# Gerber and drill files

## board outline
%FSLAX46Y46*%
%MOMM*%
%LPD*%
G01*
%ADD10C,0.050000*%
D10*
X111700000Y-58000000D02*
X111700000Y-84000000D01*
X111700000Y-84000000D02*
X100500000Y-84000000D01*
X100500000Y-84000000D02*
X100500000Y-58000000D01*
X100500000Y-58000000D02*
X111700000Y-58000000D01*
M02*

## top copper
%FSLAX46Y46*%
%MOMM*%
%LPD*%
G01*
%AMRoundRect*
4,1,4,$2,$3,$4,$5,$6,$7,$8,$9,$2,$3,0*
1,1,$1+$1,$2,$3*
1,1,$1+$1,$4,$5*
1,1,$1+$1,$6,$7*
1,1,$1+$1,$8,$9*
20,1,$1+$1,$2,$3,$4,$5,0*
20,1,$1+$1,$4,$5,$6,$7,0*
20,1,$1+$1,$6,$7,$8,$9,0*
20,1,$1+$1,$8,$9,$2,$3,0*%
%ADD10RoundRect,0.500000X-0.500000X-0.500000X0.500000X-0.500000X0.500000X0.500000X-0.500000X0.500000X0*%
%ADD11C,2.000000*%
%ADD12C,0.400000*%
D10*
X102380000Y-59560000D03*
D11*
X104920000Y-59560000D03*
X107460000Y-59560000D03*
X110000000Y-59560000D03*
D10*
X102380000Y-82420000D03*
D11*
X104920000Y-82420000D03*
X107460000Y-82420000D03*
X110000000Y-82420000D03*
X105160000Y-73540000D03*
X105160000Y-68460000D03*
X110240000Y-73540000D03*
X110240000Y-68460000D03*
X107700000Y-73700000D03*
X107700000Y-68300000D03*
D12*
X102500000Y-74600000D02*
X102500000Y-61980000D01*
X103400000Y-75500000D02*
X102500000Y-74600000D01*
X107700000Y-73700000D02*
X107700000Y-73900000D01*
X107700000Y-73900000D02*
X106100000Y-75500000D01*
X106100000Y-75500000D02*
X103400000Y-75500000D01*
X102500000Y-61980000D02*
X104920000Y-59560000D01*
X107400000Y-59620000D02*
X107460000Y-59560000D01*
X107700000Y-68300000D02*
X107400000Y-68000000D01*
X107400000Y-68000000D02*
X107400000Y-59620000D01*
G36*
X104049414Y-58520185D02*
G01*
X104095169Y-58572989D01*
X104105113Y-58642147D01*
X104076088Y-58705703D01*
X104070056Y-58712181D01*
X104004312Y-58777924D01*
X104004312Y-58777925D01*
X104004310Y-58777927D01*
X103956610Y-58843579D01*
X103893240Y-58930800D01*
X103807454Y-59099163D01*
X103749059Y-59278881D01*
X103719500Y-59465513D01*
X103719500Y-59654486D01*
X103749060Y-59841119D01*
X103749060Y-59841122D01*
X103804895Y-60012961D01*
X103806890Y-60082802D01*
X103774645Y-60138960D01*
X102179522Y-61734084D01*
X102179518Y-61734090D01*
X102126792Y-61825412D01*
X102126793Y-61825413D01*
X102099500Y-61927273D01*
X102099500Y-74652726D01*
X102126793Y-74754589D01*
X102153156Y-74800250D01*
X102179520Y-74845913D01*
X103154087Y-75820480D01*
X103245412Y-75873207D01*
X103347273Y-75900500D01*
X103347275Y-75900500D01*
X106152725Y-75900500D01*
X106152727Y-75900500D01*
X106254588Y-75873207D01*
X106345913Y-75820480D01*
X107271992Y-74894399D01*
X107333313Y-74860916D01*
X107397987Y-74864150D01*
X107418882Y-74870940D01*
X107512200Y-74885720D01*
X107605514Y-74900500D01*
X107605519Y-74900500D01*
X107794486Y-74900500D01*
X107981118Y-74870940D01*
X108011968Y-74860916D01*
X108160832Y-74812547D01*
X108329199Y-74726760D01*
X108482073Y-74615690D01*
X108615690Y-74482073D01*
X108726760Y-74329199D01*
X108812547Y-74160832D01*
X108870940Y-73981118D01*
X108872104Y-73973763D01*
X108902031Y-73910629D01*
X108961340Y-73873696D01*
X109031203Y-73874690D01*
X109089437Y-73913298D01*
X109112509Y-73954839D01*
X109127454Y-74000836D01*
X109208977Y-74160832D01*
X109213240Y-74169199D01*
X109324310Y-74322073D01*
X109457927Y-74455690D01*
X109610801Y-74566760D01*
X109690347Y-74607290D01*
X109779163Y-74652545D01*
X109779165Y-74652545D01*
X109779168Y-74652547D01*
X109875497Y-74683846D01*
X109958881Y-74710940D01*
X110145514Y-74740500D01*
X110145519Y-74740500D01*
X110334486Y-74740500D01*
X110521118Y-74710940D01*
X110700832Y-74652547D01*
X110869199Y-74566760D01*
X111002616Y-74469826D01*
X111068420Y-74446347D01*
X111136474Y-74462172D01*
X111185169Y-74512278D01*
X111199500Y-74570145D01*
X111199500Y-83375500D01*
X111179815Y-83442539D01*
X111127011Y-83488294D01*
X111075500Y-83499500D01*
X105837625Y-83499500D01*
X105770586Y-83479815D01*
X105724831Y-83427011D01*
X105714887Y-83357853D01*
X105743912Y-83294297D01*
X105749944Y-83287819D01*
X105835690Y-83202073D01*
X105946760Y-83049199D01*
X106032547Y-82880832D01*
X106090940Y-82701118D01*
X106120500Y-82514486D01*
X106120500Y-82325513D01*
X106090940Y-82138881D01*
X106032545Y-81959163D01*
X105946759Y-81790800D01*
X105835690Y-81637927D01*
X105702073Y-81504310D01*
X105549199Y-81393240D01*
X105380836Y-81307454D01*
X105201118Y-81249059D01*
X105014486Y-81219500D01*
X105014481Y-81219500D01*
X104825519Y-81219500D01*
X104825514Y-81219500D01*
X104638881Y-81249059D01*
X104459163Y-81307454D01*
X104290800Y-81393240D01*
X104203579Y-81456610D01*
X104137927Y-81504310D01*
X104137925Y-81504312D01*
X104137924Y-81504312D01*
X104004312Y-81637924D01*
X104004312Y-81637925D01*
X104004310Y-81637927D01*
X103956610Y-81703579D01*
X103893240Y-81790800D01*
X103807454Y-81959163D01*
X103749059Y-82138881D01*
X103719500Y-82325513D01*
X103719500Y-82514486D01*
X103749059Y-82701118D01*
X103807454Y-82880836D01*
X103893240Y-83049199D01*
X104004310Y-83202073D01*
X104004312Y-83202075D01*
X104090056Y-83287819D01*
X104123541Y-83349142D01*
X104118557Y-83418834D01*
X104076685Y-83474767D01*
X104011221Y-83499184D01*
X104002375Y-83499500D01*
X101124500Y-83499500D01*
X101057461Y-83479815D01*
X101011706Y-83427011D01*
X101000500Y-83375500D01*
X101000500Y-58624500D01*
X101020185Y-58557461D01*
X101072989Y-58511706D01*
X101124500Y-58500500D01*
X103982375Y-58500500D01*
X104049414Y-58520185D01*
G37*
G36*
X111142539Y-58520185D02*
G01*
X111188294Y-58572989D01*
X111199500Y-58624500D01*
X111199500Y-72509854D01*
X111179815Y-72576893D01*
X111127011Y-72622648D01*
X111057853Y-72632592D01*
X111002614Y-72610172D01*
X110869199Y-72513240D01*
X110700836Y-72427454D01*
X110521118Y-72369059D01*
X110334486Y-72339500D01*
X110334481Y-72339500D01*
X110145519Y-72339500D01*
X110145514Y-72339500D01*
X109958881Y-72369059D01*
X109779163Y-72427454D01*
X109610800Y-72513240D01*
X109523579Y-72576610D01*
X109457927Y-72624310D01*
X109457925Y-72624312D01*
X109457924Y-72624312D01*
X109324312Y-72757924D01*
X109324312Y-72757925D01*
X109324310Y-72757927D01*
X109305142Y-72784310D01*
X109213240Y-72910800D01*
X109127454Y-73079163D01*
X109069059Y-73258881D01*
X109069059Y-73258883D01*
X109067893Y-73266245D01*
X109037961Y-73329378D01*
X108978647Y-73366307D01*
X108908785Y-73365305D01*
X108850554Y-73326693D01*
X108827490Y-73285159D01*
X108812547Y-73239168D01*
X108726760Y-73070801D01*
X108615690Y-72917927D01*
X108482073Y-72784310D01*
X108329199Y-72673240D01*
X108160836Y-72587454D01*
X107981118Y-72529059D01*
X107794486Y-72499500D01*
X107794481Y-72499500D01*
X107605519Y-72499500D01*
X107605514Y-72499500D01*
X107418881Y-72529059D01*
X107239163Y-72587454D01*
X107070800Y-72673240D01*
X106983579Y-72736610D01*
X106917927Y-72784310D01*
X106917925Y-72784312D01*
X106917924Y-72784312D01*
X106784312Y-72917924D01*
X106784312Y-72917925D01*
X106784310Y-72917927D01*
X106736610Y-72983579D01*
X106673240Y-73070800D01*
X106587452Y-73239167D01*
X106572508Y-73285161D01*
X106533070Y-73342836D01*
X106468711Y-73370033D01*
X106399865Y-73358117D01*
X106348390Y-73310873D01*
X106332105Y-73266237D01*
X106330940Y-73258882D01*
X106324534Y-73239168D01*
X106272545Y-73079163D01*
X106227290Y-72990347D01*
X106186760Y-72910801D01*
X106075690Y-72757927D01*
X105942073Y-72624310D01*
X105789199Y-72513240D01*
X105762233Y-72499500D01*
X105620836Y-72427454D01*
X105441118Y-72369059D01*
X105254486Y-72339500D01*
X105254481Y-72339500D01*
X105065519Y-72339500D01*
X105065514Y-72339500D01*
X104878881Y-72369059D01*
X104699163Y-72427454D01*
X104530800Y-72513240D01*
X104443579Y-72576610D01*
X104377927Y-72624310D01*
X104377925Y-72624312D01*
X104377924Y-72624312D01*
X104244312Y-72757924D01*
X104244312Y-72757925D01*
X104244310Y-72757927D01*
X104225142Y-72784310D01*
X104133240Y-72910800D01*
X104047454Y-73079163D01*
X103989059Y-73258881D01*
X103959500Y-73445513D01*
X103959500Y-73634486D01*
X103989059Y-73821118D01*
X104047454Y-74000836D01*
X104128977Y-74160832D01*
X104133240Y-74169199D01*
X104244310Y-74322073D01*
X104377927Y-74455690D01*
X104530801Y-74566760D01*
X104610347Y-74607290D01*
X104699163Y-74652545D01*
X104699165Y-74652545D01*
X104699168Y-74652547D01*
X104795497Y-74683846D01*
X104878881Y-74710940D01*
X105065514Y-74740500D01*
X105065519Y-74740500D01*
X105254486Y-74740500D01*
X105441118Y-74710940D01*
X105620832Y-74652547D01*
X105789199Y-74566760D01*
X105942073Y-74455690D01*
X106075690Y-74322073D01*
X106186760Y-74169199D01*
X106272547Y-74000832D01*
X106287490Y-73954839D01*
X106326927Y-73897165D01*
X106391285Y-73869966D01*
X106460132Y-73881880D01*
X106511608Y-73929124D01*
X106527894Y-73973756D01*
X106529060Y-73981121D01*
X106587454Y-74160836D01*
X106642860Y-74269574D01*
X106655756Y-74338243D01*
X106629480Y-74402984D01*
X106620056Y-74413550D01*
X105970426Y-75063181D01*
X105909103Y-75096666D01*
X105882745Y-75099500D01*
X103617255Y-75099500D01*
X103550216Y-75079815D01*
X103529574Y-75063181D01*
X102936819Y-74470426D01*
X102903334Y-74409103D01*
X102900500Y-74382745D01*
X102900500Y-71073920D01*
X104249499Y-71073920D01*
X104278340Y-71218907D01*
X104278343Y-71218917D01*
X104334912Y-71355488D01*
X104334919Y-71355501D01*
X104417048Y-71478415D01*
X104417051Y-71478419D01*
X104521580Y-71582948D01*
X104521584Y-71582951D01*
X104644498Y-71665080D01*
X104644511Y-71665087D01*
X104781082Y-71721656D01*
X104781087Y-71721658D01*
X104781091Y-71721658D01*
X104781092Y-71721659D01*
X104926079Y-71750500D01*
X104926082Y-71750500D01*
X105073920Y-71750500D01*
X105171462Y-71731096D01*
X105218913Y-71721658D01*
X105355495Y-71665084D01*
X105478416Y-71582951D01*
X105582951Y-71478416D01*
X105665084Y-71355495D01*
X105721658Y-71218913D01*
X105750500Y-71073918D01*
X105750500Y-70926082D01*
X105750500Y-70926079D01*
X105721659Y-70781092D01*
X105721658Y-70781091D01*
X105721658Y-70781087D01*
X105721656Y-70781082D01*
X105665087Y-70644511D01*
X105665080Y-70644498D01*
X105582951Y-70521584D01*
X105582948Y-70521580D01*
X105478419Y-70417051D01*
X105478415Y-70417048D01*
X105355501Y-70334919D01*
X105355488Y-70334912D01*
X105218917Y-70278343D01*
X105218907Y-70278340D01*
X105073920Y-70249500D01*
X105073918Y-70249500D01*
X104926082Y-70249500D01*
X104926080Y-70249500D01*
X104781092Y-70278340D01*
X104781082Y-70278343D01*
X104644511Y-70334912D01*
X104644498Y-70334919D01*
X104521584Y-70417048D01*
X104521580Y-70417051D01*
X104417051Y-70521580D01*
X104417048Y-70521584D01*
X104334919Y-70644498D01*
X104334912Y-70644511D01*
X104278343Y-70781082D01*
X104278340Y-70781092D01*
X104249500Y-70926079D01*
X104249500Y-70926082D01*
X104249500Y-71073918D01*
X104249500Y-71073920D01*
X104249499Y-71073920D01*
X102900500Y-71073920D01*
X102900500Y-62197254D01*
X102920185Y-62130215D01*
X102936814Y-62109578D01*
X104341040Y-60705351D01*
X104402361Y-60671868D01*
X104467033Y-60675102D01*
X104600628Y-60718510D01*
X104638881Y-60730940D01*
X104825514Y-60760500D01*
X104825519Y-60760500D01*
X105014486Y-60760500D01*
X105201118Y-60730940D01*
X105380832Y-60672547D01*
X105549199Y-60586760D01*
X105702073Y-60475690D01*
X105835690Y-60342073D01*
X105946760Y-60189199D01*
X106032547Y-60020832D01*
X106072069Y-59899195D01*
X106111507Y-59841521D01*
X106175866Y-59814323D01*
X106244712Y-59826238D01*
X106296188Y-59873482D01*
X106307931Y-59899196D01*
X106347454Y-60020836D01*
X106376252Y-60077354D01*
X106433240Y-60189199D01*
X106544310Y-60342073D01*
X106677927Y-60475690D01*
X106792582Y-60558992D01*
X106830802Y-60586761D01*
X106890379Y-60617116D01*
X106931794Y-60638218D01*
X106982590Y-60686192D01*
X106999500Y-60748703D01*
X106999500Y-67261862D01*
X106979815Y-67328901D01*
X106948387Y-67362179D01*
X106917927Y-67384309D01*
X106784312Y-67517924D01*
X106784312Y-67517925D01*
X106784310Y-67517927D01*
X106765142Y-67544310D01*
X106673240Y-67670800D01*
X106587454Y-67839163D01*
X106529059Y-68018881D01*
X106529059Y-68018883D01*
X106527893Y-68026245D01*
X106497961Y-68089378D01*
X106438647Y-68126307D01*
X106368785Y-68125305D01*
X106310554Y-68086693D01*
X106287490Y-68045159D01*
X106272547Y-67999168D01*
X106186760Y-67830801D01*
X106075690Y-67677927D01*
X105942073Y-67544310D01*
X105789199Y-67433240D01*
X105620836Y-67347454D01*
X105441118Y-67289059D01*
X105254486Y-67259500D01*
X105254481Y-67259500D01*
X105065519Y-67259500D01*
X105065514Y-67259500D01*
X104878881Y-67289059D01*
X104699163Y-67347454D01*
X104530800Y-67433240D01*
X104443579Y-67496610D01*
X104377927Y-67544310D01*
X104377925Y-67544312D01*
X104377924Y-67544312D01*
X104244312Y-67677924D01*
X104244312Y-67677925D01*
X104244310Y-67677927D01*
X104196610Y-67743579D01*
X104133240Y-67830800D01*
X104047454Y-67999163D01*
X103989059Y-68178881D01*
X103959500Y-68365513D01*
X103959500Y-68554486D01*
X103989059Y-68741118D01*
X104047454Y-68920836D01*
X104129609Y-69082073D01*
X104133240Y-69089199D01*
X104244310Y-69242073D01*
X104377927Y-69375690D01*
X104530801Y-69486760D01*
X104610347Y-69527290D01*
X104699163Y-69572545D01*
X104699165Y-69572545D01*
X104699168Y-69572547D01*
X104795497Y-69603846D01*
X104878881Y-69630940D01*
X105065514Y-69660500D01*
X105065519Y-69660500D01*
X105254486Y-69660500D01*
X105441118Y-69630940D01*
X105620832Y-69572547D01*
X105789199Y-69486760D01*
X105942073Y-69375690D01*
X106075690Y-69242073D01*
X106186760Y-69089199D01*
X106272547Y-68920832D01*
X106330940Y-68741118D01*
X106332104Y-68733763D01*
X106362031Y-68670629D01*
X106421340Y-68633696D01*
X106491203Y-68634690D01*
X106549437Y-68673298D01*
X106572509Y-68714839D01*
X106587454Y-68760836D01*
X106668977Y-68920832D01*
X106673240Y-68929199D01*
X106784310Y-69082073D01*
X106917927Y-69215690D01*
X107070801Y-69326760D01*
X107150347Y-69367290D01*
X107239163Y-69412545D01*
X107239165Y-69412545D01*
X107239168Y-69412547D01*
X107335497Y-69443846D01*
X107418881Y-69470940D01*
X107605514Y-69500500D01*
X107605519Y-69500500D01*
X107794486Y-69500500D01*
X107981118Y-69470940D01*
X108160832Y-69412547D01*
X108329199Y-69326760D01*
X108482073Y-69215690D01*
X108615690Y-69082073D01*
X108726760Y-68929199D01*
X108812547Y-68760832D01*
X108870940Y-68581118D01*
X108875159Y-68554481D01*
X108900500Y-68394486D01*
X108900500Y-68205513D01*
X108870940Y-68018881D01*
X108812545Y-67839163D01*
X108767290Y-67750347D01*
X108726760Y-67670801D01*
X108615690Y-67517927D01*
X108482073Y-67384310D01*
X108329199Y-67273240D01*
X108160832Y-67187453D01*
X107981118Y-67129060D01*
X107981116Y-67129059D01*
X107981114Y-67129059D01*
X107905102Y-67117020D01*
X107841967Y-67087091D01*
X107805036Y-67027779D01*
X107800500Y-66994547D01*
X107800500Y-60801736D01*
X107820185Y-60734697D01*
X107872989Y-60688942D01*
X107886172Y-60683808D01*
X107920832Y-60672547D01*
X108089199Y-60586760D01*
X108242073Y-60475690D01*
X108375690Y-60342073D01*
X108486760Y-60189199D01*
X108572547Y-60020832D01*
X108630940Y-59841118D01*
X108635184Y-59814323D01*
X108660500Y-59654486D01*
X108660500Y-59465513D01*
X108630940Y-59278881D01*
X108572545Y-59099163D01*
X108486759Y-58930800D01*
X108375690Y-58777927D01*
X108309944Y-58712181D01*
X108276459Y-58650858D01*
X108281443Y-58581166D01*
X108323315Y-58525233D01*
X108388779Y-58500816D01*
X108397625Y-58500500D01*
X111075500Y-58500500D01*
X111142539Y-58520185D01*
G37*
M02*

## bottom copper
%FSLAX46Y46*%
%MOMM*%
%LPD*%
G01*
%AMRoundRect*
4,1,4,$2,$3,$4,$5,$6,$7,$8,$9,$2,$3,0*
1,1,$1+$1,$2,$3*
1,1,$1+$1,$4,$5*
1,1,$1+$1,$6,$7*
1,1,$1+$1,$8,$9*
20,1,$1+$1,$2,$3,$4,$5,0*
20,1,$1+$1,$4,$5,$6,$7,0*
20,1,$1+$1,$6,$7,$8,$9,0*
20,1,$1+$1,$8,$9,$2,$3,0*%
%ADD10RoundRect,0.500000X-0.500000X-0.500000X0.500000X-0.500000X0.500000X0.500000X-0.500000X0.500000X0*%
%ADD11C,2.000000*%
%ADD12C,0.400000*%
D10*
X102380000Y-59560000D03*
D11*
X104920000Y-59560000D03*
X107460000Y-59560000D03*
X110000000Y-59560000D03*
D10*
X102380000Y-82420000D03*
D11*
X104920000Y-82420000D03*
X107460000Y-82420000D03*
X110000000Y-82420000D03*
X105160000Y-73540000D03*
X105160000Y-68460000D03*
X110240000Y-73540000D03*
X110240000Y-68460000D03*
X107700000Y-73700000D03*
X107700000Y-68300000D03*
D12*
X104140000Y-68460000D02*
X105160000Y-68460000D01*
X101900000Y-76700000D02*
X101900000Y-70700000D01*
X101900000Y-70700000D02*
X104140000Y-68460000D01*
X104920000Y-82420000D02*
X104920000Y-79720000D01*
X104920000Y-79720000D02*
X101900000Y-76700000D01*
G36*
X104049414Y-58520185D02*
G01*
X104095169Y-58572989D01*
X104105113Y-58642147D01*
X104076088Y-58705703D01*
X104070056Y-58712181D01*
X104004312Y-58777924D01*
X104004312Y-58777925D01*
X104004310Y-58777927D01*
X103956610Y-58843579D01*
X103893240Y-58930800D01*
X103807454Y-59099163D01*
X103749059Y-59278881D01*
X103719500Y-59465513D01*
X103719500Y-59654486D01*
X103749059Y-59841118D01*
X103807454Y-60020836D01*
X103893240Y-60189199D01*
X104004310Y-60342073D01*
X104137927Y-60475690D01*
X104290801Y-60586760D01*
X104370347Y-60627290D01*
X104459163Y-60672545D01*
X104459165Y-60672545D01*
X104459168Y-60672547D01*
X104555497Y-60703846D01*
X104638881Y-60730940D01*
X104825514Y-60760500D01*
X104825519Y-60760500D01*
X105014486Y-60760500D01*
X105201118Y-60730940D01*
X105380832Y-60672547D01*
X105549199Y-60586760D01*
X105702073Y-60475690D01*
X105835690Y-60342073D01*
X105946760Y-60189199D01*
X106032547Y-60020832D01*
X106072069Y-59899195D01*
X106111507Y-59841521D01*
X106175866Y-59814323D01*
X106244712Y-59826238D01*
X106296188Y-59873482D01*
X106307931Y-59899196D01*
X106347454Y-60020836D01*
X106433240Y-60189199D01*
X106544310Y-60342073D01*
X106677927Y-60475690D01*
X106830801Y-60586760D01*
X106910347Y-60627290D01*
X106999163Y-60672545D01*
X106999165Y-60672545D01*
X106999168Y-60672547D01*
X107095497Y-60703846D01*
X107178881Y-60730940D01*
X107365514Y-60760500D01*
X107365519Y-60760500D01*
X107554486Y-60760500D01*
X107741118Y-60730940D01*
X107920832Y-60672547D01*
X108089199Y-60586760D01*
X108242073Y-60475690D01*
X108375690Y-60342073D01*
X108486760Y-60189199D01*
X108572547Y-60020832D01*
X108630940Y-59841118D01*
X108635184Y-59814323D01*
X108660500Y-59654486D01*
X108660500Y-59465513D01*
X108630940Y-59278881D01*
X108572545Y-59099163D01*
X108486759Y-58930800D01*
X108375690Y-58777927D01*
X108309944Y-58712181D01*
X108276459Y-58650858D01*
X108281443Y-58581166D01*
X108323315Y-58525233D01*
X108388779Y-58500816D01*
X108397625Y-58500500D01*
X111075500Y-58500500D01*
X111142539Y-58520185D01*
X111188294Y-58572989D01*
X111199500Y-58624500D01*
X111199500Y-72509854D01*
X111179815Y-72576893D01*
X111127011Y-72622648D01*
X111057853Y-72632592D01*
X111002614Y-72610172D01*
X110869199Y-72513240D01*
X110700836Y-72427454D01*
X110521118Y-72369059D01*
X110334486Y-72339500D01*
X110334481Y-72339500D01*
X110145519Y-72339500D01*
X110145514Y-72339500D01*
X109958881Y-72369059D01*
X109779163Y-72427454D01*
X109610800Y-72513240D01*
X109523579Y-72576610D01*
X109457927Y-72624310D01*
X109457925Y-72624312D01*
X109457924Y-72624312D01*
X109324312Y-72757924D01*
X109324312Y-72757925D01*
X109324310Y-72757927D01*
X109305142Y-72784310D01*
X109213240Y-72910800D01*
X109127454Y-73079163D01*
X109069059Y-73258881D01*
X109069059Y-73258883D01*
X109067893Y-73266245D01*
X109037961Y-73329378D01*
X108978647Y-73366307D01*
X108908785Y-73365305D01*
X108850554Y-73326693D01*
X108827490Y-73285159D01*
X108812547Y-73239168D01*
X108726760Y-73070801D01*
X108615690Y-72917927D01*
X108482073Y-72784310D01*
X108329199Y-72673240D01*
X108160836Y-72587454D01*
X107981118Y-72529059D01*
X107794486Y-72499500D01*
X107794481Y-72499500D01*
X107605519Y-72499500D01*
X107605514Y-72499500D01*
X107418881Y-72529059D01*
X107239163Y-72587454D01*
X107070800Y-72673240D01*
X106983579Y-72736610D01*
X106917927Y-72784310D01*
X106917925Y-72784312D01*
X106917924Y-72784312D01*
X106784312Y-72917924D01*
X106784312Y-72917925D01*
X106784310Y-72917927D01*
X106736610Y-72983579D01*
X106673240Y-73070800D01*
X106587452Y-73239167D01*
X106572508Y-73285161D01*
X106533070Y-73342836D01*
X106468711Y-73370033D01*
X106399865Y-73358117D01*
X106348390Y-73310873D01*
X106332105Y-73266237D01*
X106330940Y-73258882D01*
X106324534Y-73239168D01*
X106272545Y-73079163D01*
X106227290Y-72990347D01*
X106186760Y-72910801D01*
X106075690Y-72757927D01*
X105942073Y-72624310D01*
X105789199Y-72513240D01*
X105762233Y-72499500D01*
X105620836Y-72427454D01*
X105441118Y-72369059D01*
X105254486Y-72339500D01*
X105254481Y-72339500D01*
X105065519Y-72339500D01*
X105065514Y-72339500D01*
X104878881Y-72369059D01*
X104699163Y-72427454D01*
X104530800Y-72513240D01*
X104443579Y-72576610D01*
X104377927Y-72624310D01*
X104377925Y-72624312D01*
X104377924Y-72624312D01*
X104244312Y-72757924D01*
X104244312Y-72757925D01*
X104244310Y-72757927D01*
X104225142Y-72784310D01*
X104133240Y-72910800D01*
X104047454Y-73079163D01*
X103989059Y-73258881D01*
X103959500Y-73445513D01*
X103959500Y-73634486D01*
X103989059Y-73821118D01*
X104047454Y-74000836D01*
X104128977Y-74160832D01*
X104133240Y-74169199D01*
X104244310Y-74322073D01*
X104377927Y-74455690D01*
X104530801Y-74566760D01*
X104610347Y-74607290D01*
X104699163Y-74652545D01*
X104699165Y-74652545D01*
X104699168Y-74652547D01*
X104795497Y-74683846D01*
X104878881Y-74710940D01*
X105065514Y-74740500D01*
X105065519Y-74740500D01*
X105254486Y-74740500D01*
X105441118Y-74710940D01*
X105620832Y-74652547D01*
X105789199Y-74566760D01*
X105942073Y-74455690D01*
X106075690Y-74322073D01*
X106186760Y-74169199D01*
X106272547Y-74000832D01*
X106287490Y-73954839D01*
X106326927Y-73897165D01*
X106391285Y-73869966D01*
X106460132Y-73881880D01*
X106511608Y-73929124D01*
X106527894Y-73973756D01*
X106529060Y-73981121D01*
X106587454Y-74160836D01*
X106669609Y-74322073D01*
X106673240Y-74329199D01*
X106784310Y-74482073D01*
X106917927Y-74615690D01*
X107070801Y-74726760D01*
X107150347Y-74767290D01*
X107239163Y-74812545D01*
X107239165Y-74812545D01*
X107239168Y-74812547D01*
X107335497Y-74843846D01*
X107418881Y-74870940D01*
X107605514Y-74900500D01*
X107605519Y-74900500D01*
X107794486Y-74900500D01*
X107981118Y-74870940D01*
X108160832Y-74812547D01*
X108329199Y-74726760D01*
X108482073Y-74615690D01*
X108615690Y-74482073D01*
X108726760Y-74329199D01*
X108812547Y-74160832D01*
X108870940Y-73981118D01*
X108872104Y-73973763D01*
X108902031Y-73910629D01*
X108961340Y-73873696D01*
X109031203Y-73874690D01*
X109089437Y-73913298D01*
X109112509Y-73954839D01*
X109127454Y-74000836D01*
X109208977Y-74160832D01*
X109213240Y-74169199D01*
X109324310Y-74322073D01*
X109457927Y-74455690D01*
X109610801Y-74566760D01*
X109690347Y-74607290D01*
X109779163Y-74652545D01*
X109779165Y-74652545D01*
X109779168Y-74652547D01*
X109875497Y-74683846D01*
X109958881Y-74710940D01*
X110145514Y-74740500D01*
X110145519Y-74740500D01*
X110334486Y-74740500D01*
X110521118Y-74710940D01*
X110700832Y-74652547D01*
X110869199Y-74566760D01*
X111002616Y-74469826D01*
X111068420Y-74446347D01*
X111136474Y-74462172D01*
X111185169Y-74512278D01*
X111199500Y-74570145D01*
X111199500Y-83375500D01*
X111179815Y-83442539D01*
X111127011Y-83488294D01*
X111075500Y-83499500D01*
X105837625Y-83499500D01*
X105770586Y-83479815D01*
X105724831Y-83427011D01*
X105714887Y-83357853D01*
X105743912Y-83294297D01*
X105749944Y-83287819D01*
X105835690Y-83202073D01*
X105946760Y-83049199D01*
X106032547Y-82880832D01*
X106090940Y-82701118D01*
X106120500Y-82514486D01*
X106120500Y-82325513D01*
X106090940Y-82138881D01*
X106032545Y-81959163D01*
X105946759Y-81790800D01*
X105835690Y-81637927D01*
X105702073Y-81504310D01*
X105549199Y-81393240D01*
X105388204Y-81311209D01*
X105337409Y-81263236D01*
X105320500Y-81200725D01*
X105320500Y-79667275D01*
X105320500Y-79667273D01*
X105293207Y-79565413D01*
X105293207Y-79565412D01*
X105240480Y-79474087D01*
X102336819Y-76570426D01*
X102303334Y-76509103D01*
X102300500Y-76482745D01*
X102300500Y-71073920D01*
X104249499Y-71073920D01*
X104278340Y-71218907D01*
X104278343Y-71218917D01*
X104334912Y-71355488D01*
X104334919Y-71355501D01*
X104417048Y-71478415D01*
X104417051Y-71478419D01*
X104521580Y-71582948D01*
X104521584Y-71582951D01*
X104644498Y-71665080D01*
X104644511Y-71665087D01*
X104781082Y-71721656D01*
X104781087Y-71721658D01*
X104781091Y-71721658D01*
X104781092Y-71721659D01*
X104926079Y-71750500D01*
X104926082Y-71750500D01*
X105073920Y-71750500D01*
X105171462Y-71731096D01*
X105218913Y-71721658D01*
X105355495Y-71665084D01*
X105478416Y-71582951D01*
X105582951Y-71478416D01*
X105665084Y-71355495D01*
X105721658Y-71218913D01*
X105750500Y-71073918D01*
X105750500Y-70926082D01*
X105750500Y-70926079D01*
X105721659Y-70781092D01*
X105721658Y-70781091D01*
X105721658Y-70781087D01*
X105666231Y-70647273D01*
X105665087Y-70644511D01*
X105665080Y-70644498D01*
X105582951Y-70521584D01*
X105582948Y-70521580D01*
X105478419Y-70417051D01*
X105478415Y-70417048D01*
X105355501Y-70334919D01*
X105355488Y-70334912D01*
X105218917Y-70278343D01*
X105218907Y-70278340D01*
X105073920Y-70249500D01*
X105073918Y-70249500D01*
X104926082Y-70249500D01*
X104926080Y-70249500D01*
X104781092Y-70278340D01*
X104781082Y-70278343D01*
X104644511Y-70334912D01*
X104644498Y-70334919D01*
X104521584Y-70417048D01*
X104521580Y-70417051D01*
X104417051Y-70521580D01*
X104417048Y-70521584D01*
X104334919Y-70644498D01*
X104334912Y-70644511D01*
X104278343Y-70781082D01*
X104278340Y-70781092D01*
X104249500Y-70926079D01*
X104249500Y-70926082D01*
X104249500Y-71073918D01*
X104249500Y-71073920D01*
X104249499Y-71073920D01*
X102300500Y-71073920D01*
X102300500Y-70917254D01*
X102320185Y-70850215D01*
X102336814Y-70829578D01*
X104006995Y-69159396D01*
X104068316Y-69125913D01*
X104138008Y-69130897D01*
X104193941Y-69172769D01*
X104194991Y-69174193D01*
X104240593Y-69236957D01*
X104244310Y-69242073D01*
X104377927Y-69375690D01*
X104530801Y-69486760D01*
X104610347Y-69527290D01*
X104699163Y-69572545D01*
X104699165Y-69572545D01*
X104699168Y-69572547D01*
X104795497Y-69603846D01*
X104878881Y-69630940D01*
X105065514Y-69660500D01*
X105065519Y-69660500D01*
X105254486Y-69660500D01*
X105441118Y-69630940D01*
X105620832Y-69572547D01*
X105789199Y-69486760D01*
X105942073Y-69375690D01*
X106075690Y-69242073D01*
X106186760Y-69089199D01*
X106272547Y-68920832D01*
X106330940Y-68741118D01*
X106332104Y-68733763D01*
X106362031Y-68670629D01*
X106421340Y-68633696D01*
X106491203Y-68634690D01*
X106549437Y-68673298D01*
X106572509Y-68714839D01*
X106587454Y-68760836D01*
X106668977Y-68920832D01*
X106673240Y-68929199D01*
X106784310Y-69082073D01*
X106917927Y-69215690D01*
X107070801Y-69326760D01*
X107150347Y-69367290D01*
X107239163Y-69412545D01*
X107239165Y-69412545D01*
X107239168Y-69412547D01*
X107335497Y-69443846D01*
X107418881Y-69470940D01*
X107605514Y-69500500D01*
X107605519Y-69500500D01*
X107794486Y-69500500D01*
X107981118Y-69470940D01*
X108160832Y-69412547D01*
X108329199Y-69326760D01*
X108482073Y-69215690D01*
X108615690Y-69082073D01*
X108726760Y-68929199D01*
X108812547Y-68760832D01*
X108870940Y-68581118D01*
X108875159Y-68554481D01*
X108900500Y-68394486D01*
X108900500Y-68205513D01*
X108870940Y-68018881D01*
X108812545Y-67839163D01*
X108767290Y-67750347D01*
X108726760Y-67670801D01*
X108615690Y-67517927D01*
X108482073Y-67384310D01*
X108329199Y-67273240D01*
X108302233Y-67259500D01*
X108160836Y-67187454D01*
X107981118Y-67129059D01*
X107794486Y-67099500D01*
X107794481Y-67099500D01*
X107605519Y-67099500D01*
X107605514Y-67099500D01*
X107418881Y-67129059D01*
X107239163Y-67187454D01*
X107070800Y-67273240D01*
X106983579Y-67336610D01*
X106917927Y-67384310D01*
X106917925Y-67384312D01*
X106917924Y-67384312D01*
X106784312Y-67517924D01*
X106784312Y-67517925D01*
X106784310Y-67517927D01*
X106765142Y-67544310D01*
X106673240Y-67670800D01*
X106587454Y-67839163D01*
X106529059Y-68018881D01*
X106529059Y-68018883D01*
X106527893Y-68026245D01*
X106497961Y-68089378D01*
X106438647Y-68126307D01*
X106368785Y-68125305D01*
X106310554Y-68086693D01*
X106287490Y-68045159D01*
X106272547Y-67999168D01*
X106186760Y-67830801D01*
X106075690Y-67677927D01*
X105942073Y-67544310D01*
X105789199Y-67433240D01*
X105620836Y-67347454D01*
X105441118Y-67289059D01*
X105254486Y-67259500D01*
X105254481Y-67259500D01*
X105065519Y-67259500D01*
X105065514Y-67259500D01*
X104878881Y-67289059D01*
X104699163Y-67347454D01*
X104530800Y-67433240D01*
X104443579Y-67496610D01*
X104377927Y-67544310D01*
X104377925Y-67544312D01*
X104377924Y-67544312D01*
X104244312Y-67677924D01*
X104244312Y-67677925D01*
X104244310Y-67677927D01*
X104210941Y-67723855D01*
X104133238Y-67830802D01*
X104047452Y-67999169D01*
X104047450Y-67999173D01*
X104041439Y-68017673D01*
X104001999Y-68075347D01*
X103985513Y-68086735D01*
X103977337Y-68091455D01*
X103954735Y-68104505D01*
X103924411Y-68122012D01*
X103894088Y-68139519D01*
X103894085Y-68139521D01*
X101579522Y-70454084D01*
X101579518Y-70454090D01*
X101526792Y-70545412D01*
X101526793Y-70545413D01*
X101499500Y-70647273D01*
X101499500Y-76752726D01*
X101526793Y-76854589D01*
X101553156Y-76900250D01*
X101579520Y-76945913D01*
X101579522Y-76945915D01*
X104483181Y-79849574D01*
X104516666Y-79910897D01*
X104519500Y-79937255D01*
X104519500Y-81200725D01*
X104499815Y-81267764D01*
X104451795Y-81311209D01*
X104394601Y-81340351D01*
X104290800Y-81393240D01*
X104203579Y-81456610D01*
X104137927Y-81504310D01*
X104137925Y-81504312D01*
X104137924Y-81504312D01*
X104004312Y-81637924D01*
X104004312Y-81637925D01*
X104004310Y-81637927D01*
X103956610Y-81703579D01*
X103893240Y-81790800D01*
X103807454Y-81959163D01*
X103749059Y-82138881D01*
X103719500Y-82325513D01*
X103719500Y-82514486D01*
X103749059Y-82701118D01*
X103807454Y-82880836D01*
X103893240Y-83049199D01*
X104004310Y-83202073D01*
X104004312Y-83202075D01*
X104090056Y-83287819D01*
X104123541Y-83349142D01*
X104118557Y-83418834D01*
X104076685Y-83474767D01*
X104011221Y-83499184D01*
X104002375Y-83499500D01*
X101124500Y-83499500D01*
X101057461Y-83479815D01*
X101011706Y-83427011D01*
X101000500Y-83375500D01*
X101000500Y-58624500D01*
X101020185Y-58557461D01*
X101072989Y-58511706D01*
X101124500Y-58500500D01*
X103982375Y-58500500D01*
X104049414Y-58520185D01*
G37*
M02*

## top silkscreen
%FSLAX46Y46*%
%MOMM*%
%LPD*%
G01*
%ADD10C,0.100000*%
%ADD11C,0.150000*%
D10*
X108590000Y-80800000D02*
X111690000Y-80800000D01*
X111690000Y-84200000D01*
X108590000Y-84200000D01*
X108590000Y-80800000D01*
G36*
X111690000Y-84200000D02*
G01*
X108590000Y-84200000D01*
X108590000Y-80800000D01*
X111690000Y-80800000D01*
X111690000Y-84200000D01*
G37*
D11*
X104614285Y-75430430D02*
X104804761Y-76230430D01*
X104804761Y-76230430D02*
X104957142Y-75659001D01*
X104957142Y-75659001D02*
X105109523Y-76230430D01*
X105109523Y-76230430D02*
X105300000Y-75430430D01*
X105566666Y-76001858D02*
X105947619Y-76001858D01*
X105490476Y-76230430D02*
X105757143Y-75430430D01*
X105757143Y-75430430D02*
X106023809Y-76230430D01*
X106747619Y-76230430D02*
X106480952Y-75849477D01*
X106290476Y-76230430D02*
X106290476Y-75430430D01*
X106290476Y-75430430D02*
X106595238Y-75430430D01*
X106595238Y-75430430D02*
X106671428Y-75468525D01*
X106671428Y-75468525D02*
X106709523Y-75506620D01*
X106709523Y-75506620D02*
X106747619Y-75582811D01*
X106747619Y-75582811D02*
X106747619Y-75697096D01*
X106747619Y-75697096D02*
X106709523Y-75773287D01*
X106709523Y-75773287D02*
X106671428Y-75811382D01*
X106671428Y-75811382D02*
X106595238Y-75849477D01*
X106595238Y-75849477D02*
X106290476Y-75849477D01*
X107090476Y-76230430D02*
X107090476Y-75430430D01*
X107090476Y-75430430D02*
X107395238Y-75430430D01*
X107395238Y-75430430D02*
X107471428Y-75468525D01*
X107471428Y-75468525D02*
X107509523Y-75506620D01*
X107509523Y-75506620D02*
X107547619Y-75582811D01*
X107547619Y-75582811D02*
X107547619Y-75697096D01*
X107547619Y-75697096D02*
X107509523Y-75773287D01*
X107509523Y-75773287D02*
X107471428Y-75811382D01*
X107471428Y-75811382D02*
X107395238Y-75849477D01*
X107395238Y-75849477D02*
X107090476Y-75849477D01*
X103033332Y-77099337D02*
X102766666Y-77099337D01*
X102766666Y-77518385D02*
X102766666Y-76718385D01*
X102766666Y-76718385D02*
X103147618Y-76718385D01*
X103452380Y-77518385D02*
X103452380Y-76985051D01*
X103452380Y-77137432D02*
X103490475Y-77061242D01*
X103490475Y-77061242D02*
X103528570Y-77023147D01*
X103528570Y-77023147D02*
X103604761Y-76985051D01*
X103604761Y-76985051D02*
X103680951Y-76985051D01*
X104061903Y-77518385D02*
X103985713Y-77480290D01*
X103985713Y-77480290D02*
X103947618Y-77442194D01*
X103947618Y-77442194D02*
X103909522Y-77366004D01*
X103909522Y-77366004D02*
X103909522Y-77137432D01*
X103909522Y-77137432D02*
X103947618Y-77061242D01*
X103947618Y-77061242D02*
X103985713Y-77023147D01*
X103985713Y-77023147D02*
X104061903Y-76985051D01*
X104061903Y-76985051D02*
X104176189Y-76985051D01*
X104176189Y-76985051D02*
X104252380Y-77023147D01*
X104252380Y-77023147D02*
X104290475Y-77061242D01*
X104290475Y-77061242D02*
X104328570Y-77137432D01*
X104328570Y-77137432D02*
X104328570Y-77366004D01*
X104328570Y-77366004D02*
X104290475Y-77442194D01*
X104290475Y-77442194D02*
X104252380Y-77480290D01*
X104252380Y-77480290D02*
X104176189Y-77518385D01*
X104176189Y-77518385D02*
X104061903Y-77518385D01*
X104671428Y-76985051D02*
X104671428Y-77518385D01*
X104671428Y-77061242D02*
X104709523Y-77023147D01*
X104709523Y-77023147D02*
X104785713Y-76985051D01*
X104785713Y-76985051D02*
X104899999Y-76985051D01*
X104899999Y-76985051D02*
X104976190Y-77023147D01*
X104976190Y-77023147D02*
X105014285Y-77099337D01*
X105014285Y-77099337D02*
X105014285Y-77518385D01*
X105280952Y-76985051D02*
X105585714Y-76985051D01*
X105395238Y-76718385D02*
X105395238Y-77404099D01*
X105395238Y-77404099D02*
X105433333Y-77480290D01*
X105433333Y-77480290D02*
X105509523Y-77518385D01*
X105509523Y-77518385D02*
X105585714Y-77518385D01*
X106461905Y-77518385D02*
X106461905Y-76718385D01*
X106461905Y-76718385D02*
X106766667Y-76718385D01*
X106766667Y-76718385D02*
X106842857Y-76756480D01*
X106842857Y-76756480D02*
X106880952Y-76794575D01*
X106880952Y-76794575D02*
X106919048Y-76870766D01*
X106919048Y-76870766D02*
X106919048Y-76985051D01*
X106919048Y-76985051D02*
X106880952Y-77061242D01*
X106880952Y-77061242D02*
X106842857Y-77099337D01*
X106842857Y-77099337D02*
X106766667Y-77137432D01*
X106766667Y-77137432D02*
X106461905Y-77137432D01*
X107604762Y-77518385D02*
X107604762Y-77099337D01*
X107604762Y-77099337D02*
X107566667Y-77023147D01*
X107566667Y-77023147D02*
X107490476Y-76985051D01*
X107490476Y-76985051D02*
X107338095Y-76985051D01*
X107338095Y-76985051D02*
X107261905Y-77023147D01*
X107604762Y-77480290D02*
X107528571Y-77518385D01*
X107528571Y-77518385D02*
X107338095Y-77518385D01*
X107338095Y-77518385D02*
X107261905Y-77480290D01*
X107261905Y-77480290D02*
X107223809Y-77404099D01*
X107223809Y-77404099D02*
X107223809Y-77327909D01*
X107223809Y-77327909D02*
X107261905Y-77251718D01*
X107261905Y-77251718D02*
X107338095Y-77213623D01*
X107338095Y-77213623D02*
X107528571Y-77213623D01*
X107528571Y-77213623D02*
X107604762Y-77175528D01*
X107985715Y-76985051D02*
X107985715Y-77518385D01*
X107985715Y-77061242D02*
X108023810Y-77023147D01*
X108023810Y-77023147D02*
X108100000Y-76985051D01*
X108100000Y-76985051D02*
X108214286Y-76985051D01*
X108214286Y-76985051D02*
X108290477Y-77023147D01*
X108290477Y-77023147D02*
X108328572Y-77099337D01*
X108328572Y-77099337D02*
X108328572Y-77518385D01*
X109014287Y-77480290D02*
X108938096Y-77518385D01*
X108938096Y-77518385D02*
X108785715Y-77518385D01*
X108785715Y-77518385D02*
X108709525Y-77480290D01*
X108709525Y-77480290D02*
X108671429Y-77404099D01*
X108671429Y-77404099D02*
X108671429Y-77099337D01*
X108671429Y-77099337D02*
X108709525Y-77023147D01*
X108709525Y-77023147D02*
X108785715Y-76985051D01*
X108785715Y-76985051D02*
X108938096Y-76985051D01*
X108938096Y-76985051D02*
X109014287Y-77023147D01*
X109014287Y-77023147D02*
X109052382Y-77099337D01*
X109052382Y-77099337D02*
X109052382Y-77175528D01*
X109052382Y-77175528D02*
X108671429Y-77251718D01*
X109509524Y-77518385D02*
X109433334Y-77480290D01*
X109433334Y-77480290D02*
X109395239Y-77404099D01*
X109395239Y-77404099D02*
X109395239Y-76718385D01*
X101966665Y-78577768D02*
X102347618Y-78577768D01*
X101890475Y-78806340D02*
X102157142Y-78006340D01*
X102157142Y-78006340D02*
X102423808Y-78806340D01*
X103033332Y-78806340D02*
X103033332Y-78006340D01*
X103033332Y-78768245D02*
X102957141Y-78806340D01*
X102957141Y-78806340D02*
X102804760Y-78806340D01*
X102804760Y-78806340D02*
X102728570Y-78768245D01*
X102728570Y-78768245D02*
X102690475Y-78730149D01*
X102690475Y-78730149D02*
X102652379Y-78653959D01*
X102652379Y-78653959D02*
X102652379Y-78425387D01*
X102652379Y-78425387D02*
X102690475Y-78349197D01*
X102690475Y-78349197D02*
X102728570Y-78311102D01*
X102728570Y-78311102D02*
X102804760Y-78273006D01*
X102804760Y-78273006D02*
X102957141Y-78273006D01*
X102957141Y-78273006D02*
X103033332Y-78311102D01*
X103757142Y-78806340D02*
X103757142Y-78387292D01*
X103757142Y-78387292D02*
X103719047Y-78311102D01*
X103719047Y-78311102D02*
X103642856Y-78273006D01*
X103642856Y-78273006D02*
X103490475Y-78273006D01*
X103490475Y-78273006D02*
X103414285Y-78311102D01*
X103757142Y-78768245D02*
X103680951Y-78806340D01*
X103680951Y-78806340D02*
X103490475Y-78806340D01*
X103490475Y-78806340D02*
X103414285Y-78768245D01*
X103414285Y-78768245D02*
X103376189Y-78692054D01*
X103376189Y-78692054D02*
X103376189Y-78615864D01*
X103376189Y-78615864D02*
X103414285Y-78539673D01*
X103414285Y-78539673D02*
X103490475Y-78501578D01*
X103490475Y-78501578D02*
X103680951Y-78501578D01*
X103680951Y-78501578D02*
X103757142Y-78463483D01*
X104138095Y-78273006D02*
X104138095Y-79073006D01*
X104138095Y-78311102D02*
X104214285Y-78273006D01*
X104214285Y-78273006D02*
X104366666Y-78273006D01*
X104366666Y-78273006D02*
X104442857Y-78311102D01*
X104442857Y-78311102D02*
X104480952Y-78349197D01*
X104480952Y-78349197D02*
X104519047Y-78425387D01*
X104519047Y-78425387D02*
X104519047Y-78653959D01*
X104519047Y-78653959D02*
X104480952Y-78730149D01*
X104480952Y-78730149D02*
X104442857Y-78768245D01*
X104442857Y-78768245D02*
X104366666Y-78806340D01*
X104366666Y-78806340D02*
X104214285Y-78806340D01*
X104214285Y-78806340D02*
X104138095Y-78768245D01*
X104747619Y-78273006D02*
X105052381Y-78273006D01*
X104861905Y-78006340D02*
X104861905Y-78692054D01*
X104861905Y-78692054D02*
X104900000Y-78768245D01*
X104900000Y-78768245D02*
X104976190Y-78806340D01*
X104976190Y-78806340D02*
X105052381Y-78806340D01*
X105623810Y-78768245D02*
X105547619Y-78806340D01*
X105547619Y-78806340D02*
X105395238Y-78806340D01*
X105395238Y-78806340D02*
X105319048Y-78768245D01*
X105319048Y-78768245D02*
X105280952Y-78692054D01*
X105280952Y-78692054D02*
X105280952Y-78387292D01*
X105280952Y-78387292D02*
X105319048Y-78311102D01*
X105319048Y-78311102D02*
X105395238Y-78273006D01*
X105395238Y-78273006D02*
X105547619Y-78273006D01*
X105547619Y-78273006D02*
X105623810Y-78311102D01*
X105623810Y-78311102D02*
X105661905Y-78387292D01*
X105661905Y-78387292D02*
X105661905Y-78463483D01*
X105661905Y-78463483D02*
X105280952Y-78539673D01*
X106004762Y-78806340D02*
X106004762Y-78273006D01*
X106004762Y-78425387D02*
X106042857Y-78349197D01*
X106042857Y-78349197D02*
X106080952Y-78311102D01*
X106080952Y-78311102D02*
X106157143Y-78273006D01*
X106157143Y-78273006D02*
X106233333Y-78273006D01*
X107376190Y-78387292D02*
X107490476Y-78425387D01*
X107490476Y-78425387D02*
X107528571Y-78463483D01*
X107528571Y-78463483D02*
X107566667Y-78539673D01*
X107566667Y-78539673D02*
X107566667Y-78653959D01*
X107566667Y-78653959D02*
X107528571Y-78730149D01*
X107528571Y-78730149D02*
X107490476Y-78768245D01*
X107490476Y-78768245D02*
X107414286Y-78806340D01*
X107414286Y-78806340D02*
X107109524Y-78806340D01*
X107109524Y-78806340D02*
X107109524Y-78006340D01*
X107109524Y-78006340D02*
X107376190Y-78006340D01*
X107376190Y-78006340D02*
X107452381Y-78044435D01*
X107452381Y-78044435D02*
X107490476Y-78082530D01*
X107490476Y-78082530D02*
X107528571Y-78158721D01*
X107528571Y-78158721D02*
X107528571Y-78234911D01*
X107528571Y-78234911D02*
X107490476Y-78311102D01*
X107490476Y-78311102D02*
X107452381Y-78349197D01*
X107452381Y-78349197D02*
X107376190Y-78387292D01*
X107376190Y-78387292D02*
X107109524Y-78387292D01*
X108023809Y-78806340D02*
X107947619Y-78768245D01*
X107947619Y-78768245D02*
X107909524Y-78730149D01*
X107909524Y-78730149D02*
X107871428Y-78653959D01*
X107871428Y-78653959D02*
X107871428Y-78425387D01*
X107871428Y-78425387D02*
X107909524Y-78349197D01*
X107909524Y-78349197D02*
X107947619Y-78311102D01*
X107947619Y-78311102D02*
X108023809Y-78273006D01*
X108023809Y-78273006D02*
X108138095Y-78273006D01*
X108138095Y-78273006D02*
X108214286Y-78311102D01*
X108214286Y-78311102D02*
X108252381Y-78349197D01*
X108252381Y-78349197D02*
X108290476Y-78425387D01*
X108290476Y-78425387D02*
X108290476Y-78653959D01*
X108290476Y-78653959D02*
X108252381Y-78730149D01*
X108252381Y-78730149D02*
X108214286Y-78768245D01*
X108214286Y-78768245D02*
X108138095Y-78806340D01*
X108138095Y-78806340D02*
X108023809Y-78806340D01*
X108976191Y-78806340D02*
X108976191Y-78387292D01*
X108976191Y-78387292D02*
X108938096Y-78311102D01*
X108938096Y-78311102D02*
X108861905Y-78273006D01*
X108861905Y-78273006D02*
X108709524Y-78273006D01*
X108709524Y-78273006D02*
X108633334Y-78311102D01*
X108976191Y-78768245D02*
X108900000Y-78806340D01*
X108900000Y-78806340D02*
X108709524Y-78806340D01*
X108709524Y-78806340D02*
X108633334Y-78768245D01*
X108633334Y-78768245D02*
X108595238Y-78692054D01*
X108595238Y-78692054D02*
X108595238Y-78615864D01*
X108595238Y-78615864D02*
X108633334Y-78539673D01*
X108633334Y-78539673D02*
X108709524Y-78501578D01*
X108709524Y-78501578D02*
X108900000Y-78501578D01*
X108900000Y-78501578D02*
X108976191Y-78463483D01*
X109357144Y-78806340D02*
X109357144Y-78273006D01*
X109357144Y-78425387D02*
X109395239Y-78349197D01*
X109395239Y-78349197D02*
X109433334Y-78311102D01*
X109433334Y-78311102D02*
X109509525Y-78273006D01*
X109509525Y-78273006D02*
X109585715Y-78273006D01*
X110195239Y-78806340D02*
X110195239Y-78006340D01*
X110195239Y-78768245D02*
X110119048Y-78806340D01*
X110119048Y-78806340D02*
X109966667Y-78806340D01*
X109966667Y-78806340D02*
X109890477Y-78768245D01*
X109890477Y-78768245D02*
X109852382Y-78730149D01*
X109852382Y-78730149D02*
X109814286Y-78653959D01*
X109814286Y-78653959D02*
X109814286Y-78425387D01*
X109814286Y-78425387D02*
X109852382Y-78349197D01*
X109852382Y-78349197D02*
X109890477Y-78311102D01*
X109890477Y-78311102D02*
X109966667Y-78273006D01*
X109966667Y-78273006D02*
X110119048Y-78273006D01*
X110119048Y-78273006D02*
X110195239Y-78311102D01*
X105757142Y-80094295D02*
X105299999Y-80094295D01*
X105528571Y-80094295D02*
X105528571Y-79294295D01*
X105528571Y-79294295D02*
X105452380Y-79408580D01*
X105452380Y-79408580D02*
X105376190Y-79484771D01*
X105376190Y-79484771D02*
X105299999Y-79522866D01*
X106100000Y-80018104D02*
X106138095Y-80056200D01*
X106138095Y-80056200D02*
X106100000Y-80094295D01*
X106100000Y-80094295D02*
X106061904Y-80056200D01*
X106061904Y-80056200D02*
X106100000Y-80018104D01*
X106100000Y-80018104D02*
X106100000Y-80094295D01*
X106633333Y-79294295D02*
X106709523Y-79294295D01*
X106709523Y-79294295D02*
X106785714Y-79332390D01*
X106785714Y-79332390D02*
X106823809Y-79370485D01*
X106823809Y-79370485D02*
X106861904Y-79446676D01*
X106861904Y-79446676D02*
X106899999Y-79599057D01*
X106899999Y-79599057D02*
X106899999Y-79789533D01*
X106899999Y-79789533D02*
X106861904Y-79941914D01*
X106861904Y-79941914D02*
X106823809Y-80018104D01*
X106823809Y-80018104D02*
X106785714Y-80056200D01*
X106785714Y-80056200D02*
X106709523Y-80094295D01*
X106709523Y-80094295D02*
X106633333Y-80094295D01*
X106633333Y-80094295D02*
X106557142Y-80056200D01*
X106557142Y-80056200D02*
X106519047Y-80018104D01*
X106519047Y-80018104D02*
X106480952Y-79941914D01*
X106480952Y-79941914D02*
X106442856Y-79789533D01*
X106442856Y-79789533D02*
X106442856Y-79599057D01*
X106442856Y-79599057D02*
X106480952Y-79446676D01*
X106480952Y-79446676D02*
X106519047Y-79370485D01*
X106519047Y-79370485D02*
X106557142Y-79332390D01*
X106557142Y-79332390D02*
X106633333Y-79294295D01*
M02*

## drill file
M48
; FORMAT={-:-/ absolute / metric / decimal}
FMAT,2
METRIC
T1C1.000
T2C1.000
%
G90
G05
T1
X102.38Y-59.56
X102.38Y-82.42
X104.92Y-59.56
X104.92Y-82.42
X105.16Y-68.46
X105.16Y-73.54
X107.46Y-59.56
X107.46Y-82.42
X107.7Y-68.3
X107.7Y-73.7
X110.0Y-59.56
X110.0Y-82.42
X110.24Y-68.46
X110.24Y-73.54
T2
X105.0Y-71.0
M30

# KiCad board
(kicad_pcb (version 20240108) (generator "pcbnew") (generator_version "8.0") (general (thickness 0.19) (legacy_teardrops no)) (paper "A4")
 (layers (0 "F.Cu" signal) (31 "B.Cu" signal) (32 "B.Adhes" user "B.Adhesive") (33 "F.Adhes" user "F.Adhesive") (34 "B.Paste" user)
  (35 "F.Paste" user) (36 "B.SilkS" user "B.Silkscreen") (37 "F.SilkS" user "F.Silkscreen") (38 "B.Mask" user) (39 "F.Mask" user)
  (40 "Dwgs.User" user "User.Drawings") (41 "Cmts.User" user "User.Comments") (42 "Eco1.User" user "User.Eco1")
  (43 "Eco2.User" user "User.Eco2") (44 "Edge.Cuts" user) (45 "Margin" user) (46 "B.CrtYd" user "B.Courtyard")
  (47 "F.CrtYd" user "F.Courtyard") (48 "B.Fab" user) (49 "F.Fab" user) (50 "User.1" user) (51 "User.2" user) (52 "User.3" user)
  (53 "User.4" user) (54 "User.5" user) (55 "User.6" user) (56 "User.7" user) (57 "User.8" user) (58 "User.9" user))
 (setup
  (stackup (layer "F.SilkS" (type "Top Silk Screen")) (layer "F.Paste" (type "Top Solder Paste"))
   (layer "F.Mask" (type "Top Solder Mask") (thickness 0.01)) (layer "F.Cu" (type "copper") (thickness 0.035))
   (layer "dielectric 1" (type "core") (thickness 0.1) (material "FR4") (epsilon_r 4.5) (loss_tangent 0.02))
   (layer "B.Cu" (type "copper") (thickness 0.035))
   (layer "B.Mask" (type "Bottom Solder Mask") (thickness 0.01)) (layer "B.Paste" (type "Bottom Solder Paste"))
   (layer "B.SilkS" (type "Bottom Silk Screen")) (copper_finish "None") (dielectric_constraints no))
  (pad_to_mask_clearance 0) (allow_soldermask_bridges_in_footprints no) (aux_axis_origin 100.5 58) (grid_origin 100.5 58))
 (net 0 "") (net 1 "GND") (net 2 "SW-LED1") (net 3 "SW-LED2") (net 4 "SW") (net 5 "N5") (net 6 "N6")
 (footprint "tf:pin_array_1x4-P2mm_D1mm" (layer "F.Cu") (at 106.19 59.56)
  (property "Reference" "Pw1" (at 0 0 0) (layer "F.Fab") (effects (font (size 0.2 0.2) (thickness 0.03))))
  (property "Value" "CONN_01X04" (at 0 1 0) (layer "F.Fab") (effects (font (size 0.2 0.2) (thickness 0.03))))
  (pad "1" thru_hole roundrect (at -3.81 0) (size 2 2) (drill 1) (layers "*.Cu" "*.Mask") (remove_unused_layers no) (roundrect_rratio 0.25)
   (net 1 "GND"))
  (pad "2" thru_hole circle (at -1.27 0) (size 2 2) (drill 1) (layers "*.Cu" "*.Mask") (remove_unused_layers no) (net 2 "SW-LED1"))
  (pad "3" thru_hole circle (at 1.27 0) (size 2 2) (drill 1) (layers "*.Cu" "*.Mask") (remove_unused_layers no) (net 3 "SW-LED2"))
  (pad "4" thru_hole circle (at 3.81 0) (size 2 2) (drill 1) (layers "*.Cu" "*.Mask") (remove_unused_layers no) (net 1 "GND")))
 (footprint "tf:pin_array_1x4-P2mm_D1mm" (layer "F.Cu") (at 106.19 82.42)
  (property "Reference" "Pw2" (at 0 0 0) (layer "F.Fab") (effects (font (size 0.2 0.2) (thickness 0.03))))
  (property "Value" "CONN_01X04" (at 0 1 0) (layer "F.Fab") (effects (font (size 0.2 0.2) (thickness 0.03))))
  (pad "1" thru_hole roundrect (at -3.81 0) (size 2 2) (drill 1) (layers "*.Cu" "*.Mask") (remove_unused_layers no) (roundrect_rratio 0.25)
   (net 1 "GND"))
  (pad "2" thru_hole circle (at -1.27 0) (size 2 2) (drill 1) (layers "*.Cu" "*.Mask") (remove_unused_layers no) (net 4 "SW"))
  (pad "3" thru_hole circle (at 1.27 0) (size 2 2) (drill 1) (layers "*.Cu" "*.Mask") (remove_unused_layers no) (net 1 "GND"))
  (pad "4" thru_hole circle (at 3.81 0) (size 2 2) (drill 1) (layers "*.Cu" "*.Mask") (remove_unused_layers no) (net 1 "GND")))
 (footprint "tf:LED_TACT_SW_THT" (layer "B.Cu") (at 107.7 71)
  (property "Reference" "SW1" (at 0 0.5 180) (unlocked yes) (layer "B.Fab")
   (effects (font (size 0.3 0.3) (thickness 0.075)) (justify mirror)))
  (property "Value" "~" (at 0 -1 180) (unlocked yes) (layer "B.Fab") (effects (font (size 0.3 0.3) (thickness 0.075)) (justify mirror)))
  (pad "" np_thru_hole circle (at -2.7 0) (size 0.1 0.1) (drill 1) (layers "F&B.Cu" "*.Mask"))
  (pad "1" thru_hole circle (at -2.54 2.54) (size 2 2) (drill 1) (layers "*.Cu" "*.Mask") (remove_unused_layers no) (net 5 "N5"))
  (pad "2" thru_hole circle (at -2.54 -2.54) (size 2 2) (drill 1) (layers "*.Cu" "*.Mask") (remove_unused_layers no) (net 4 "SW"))
  (pad "3" thru_hole circle (at 2.54 2.54) (size 2 2) (drill 1) (layers "*.Cu" "*.Mask") (remove_unused_layers no) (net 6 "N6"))
  (pad "4" thru_hole circle (at 2.54 -2.54) (size 2 2) (drill 1) (layers "*.Cu" "*.Mask") (remove_unused_layers no) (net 1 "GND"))
  (pad "L1" thru_hole circle (at 0 2.7) (size 2 2) (drill 1) (layers "*.Cu" "*.Mask") (remove_unused_layers no) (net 2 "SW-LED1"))
  (pad "L2" thru_hole circle (at 0 -2.7) (size 2 2) (drill 1) (layers "*.Cu" "*.Mask") (remove_unused_layers no) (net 3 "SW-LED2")))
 (gr_poly
  (pts (xy 108.59 80.8) (xy 111.69 80.8) (xy 111.69 84.2) (xy 108.59 84.2)) (stroke (width 0.1) (type solid)) (fill solid) (layer "F.SilkS"))
 (gr_line (start 111.7 58) (end 111.7 84) (stroke (width 0.05) (type default)) (layer "Edge.Cuts"))
 (gr_line (start 111.7 84) (end 100.5 84) (stroke (width 0.05) (type default)) (layer "Edge.Cuts"))
 (gr_line (start 100.5 84) (end 100.5 58) (stroke (width 0.05) (type default)) (layer "Edge.Cuts"))
 (gr_line (start 100.5 58) (end 111.7 58) (stroke (width 0.05) (type default)) (layer "Edge.Cuts"))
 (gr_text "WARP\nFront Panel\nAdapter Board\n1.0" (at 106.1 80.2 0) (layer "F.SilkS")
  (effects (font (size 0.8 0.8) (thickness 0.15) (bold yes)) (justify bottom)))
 (segment (start 102.5 74.6) (end 102.5 61.98) (width 0.4) (layer "F.Cu") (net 2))
 (segment (start 103.4 75.5) (end 102.5 74.6) (width 0.4) (layer "F.Cu") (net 2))
 (segment (start 107.7 73.7) (end 107.7 73.9) (width 0.4) (layer "F.Cu") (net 2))
 (segment (start 107.7 73.9) (end 106.1 75.5) (width 0.4) (layer "F.Cu") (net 2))
 (segment (start 106.1 75.5) (end 103.4 75.5) (width 0.4) (layer "F.Cu") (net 2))
 (segment (start 102.5 61.98) (end 104.92 59.56) (width 0.4) (layer "F.Cu") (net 2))
 (segment (start 107.4 59.62) (end 107.46 59.56) (width 0.4) (layer "F.Cu") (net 3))
 (segment (start 107.7 68.3) (end 107.4 68) (width 0.4) (layer "F.Cu") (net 3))
 (segment (start 107.4 68) (end 107.4 59.62) (width 0.4) (layer "F.Cu") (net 3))
 (segment (start 104.14 68.46) (end 105.16 68.46) (width 0.4) (layer "B.Cu") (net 4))
 (segment (start 101.9 76.7) (end 101.9 70.7) (width 0.4) (layer "B.Cu") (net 4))
 (segment (start 101.9 70.7) (end 104.14 68.46) (width 0.4) (layer "B.Cu") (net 4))
 (segment (start 104.92 82.42) (end 104.92 79.72) (width 0.4) (layer "B.Cu") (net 4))
 (segment (start 104.92 79.72) (end 101.9 76.7) (width 0.4) (layer "B.Cu") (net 4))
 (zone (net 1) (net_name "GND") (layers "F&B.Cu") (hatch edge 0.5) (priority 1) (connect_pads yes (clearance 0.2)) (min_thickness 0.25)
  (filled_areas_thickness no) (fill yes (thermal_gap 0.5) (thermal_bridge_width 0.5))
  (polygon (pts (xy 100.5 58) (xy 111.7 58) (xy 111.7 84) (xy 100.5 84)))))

